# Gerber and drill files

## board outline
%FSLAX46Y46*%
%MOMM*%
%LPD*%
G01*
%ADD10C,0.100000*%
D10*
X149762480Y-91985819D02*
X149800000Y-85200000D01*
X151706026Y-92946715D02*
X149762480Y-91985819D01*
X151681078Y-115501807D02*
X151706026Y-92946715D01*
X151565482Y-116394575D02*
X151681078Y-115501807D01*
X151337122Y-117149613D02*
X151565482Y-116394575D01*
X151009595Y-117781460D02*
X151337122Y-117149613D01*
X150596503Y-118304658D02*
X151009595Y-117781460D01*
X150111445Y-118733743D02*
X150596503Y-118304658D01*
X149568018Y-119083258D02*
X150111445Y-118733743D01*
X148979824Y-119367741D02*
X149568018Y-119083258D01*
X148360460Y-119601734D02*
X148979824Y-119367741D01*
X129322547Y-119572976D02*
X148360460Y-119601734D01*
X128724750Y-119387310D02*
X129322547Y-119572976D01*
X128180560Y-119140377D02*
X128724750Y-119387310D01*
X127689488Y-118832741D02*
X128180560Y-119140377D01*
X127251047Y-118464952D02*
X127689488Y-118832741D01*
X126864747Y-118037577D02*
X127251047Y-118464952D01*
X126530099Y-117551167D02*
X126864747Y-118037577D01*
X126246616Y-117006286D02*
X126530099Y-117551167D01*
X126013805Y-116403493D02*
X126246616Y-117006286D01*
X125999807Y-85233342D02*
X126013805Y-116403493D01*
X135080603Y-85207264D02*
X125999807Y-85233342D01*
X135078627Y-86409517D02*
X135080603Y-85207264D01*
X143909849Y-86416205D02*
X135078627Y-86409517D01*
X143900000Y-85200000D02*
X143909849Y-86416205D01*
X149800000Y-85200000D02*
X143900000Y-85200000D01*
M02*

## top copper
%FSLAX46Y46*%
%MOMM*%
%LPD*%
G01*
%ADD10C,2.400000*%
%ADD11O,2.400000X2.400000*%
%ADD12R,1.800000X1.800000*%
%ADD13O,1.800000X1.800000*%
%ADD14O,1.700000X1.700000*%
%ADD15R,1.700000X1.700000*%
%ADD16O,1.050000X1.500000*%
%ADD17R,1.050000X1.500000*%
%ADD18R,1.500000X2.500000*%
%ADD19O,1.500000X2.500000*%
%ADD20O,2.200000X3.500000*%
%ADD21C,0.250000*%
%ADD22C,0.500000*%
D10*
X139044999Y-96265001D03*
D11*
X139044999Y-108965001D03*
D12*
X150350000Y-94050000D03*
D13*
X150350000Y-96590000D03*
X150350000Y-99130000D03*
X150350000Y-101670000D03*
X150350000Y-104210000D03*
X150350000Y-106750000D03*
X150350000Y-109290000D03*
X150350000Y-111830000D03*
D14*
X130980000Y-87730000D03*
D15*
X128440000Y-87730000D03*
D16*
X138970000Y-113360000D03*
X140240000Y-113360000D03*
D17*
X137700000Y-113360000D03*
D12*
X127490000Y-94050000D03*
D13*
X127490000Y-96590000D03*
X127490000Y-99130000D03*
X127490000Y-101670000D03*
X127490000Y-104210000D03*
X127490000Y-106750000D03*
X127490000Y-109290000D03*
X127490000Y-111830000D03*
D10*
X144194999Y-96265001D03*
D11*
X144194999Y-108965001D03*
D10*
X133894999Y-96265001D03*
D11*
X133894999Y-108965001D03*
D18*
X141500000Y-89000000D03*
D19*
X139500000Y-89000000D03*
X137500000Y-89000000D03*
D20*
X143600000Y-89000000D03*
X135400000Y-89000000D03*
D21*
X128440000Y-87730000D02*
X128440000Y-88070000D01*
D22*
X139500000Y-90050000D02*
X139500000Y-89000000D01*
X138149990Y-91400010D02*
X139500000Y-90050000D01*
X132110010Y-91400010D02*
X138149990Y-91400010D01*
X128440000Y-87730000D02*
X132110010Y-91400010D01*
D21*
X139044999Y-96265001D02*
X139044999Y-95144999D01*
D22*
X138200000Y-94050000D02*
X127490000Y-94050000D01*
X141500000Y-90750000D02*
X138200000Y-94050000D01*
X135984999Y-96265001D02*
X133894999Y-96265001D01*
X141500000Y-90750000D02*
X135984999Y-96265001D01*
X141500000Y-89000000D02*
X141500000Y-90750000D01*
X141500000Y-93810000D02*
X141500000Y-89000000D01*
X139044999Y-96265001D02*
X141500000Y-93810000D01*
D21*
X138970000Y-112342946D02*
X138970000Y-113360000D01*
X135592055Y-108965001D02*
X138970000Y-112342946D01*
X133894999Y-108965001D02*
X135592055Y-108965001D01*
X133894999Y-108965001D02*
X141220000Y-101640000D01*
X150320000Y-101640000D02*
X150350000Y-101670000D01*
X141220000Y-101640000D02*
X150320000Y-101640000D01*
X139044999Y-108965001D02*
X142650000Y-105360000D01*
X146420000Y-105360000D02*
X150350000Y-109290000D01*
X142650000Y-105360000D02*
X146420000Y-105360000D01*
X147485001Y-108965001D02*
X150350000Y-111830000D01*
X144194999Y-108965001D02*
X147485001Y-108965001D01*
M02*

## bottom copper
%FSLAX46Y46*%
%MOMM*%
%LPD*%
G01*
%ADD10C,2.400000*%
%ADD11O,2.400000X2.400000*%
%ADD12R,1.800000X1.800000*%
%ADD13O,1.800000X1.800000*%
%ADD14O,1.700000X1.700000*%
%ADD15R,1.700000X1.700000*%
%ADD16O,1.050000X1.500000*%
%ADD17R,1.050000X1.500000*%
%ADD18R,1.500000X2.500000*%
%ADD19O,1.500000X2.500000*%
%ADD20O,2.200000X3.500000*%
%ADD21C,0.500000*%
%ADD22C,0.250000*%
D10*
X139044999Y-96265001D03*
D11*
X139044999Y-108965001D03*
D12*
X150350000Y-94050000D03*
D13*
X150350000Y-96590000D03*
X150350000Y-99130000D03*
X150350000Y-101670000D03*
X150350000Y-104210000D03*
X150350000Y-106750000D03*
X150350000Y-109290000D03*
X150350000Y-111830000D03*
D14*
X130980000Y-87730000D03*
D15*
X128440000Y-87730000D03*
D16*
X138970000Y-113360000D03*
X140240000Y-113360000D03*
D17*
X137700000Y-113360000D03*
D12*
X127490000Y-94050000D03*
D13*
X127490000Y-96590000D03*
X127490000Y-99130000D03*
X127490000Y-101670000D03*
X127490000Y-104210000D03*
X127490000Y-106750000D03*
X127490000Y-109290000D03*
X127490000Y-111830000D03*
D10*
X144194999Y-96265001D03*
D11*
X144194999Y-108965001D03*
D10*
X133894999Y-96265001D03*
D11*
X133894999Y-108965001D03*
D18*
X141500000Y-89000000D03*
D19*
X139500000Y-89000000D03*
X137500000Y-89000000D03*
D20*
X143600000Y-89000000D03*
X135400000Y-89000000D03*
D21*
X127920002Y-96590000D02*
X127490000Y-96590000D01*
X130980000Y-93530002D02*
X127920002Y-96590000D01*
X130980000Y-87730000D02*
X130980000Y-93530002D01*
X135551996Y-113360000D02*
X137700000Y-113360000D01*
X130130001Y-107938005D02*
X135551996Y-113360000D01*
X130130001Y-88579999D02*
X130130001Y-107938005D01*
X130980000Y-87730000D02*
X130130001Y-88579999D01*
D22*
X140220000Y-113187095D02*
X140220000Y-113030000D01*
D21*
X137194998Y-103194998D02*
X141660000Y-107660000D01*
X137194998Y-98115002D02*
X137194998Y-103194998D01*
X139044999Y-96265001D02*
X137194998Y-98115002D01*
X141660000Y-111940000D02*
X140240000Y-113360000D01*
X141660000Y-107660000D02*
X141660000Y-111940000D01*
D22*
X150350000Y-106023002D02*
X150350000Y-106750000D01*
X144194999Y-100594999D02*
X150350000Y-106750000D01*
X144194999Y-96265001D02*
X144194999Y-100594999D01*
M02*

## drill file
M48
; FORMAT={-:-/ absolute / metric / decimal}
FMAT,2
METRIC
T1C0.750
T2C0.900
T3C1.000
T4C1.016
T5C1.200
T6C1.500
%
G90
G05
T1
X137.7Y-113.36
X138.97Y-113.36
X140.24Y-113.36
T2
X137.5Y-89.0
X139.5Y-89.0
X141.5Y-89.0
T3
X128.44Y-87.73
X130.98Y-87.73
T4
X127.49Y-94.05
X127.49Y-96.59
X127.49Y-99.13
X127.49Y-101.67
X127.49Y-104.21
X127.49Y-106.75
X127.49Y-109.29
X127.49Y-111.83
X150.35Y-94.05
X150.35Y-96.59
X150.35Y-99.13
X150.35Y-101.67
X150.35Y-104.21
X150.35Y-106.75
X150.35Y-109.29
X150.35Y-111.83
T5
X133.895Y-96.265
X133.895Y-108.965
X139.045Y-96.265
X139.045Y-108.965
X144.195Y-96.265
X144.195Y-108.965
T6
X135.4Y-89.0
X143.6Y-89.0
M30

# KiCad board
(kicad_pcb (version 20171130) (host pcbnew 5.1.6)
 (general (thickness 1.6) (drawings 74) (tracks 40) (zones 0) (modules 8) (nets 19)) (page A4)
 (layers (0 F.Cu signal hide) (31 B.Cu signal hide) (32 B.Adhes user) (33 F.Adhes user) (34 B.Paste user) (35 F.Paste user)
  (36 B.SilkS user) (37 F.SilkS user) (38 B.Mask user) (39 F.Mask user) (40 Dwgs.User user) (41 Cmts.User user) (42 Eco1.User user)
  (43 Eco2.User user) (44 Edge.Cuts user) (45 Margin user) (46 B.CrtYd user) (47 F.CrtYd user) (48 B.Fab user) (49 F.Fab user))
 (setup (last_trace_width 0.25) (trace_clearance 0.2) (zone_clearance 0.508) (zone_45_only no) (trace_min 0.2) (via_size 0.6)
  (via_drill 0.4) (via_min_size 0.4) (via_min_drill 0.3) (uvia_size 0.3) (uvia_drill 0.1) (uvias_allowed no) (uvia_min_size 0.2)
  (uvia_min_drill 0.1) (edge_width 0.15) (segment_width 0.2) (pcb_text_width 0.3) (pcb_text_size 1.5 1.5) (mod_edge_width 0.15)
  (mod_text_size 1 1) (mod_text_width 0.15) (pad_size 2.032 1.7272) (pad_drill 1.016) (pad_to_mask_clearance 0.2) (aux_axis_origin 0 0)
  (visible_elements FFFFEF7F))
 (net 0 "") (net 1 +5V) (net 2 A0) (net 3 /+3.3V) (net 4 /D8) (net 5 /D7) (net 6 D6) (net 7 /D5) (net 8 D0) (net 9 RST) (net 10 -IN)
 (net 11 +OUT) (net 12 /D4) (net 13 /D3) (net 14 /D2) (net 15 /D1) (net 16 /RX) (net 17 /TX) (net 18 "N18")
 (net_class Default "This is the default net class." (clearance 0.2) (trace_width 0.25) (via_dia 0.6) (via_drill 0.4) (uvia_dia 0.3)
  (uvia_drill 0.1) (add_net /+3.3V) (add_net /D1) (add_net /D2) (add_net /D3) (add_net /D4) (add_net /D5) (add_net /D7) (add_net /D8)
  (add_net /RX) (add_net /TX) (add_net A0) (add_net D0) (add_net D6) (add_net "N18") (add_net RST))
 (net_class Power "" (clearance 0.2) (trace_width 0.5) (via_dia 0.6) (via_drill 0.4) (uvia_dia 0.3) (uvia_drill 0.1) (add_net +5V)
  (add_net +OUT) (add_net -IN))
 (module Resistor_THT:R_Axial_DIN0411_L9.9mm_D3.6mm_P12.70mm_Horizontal (layer F.Cu) (at 139.044999 96.265001 270)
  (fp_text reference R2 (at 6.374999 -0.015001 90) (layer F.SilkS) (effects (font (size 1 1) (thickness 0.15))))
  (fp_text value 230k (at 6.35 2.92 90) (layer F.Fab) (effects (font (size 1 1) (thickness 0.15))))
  (pad 1 thru_hole circle (at 0 0 270) (size 2.4 2.4) (drill 1.2) (layers *.Cu *.Mask) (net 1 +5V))
  (pad 2 thru_hole oval (at 12.7 0 270) (size 2.4 2.4) (drill 1.2) (layers *.Cu *.Mask) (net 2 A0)))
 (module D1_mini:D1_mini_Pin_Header (layer B.Cu) (at 150.35 94.05 180)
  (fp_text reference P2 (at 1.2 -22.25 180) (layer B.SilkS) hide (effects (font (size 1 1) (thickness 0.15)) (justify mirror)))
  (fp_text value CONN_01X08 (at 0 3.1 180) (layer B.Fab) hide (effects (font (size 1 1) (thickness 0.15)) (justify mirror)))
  (pad 1 thru_hole rect (at 0 0 180) (size 1.8 1.8) (drill 1.016) (layers *.Cu *.Mask B.SilkS) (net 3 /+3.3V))
  (pad 2 thru_hole oval (at 0 -2.54 180) (size 1.8 1.8) (drill 1.016) (layers *.Cu *.Mask B.SilkS) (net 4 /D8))
  (pad 3 thru_hole oval (at 0 -5.08 180) (size 1.8 1.8) (drill 1.016) (layers *.Cu *.Mask B.SilkS) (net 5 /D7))
  (pad 4 thru_hole oval (at 0 -7.62 180) (size 1.8 1.8) (drill 1.016) (layers *.Cu *.Mask B.SilkS) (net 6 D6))
  (pad 5 thru_hole oval (at 0 -10.16 180) (size 1.8 1.8) (drill 1.016) (layers *.Cu *.Mask B.SilkS) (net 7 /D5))
  (pad 6 thru_hole oval (at 0 -12.7 180) (size 1.8 1.8) (drill 1.016) (layers *.Cu *.Mask B.SilkS) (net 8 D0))
  (pad 7 thru_hole oval (at 0 -15.24 180) (size 1.8 1.8) (drill 1.016) (layers *.Cu *.Mask B.SilkS) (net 2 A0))
  (pad 8 thru_hole oval (at 0 -17.78 180) (size 1.8 1.8) (drill 1.016) (layers *.Cu *.Mask B.SilkS) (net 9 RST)))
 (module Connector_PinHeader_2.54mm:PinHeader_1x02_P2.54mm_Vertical (layer F.Cu) (at 128.44 87.73 90)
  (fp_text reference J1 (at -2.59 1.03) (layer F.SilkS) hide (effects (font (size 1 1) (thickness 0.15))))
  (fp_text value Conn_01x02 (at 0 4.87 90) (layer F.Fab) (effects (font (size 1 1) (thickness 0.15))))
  (pad 2 thru_hole oval (at 0 2.54 90) (size 1.7 1.7) (drill 1) (layers *.Cu *.Mask) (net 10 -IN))
  (pad 1 thru_hole rect (at 0 0 90) (size 1.7 1.7) (drill 1) (layers *.Cu *.Mask) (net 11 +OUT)))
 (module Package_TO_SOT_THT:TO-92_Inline (layer F.Cu) (at 137.7 113.36)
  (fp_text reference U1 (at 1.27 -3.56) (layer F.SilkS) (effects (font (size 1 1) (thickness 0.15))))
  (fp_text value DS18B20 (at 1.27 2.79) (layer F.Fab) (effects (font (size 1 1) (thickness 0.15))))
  (pad 2 thru_hole oval (at 1.27 0) (size 1.05 1.5) (drill 0.75) (layers *.Cu *.Mask) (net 6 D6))
  (pad 3 thru_hole oval (at 2.54 0) (size 1.05 1.5) (drill 0.75) (layers *.Cu *.Mask) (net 1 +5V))
  (pad 1 thru_hole rect (at 0 0) (size 1.05 1.5) (drill 0.75) (layers *.Cu *.Mask) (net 10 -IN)))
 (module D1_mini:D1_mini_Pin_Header (layer B.Cu) (at 127.49 94.05 180)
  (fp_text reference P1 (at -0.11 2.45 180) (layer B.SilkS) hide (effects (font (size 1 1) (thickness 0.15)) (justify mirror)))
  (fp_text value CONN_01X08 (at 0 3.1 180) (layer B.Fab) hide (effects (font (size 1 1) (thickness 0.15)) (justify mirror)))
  (pad 1 thru_hole rect (at 0 0 180) (size 1.8 1.8) (drill 1.016) (layers *.Cu *.Mask B.SilkS) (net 1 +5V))
  (pad 2 thru_hole oval (at 0 -2.54 180) (size 1.8 1.8) (drill 1.016) (layers *.Cu *.Mask B.SilkS) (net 10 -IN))
  (pad 3 thru_hole oval (at 0 -5.08 180) (size 1.8 1.8) (drill 1.016) (layers *.Cu *.Mask B.SilkS) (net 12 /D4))
  (pad 4 thru_hole oval (at 0 -7.62 180) (size 1.8 1.8) (drill 1.016) (layers *.Cu *.Mask B.SilkS) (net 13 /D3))
  (pad 5 thru_hole oval (at 0 -10.16 180) (size 1.8 1.8) (drill 1.016) (layers *.Cu *.Mask B.SilkS) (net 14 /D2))
  (pad 6 thru_hole oval (at 0 -12.7 180) (size 1.8 1.8) (drill 1.016) (layers *.Cu *.Mask B.SilkS) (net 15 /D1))
  (pad 7 thru_hole oval (at 0 -15.24 180) (size 1.8 1.8) (drill 1.016) (layers *.Cu *.Mask B.SilkS) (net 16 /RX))
  (pad 8 thru_hole oval (at 0 -17.78 180) (size 1.8 1.8) (drill 1.016) (layers *.Cu *.Mask B.SilkS) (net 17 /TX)))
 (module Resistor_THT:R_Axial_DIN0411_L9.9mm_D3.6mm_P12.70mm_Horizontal (layer F.Cu) (at 144.194999 96.265001 270)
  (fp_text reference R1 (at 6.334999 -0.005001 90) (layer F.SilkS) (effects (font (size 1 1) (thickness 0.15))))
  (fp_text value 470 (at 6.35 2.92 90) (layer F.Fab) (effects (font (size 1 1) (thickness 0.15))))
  (pad 1 thru_hole circle (at 0 0 270) (size 2.4 2.4) (drill 1.2) (layers *.Cu *.Mask) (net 8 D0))
  (pad 2 thru_hole oval (at 12.7 0 270) (size 2.4 2.4) (drill 1.2) (layers *.Cu *.Mask) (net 9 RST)))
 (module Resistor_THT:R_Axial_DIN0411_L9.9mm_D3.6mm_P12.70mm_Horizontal (layer F.Cu) (at 133.894999 96.265001 270)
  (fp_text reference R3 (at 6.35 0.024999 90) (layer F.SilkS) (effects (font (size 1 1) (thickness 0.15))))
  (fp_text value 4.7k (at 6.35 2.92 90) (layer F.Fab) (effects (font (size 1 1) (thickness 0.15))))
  (pad 1 thru_hole circle (at 0 0 270) (size 2.4 2.4) (drill 1.2) (layers *.Cu *.Mask) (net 1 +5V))
  (pad 2 thru_hole oval (at 12.7 0 270) (size 2.4 2.4) (drill 1.2) (layers *.Cu *.Mask) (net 6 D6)))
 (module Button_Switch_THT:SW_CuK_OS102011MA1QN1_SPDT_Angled (layer F.Cu) (at 141.5 89 180)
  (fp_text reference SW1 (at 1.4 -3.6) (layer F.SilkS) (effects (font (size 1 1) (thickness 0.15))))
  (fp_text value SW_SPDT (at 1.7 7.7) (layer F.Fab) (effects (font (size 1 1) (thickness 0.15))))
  (pad 1 thru_hole rect (at 0 0 180) (size 1.5 2.5) (drill 0.9) (layers *.Cu *.Mask) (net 1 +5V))
  (pad 2 thru_hole oval (at 2 0 180) (size 1.5 2.5) (drill 0.9) (layers *.Cu *.Mask) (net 11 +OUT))
  (pad 3 thru_hole oval (at 4 0 180) (size 1.5 2.5) (drill 0.9) (layers *.Cu *.Mask) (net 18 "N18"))
  (pad "" thru_hole oval (at -2.1 0 180) (size 2.2 3.5) (drill 1.5) (layers *.Cu *.Mask))
  (pad "" thru_hole oval (at 6.1 0 180) (size 2.2 3.5) (drill 1.5) (layers *.Cu *.Mask)))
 (gr_line (start 149.76248 91.985819) (end 149.8 85.2) (layer Edge.Cuts) (width 0.1))
 (gr_line (start 151.706026 92.946715) (end 149.76248 91.985819) (layer Edge.Cuts) (width 0.1))
 (gr_line (start 151.681078 115.501807) (end 151.706026 92.946715) (layer Edge.Cuts) (width 0.1))
 (gr_line (start 151.565482 116.394575) (end 151.681078 115.501807) (layer Edge.Cuts) (width 0.1))
 (gr_line (start 151.337122 117.149613) (end 151.565482 116.394575) (layer Edge.Cuts) (width 0.1))
 (gr_line (start 151.009595 117.78146) (end 151.337122 117.149613) (layer Edge.Cuts) (width 0.1))
 (gr_line (start 150.596503 118.304658) (end 151.009595 117.78146) (layer Edge.Cuts) (width 0.1))
 (gr_line (start 150.111445 118.733743) (end 150.596503 118.304658) (layer Edge.Cuts) (width 0.1))
 (gr_line (start 149.568018 119.083258) (end 150.111445 118.733743) (layer Edge.Cuts) (width 0.1))
 (gr_line (start 148.979824 119.367741) (end 149.568018 119.083258) (layer Edge.Cuts) (width 0.1))
 (gr_line (start 148.36046 119.601734) (end 148.979824 119.367741) (layer Edge.Cuts) (width 0.1))
 (gr_line (start 129.322547 119.572976) (end 148.36046 119.601734) (layer Edge.Cuts) (width 0.1))
 (gr_line (start 128.72475 119.38731) (end 129.322547 119.572976) (layer Edge.Cuts) (width 0.1))
 (gr_line (start 128.18056 119.140377) (end 128.72475 119.38731) (layer Edge.Cuts) (width 0.1))
 (gr_line (start 127.689488 118.832741) (end 128.18056 119.140377) (layer Edge.Cuts) (width 0.1))
 (gr_line (start 127.251047 118.464952) (end 127.689488 118.832741) (layer Edge.Cuts) (width 0.1))
 (gr_line (start 126.864747 118.037577) (end 127.251047 118.464952) (layer Edge.Cuts) (width 0.1))
 (gr_line (start 126.530099 117.551167) (end 126.864747 118.037577) (layer Edge.Cuts) (width 0.1))
 (gr_line (start 126.246616 117.006286) (end 126.530099 117.551167) (layer Edge.Cuts) (width 0.1))
 (gr_line (start 126.013805 116.403493) (end 126.246616 117.006286) (layer Edge.Cuts) (width 0.1))
 (gr_line (start 125.999807 85.233342) (end 126.013805 116.403493) (layer Edge.Cuts) (width 0.1))
 (gr_line (start 135.080603 85.207264) (end 125.999807 85.233342) (layer Edge.Cuts) (width 0.1))
 (gr_line (start 135.078627 86.409517) (end 135.080603 85.207264) (layer Edge.Cuts) (width 0.1))
 (gr_line (start 143.909849 86.416205) (end 135.078627 86.409517) (layer Edge.Cuts) (width 0.1))
 (gr_line (start 143.9 85.2) (end 143.909849 86.416205) (layer Edge.Cuts) (width 0.1))
 (gr_line (start 149.8 85.2) (end 143.9 85.2) (layer Edge.Cuts) (width 0.1))
 (segment (start 128.44 87.73) (end 128.44 88.07) (width 0.25) (layer F.Cu) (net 11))
 (segment (start 139.5 90.05) (end 139.5 89) (width 0.5) (layer F.Cu) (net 11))
 (segment (start 138.14999 91.40001) (end 139.5 90.05) (width 0.5) (layer F.Cu) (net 11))
 (segment (start 132.11001 91.40001) (end 138.14999 91.40001) (width 0.5) (layer F.Cu) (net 11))
 (segment (start 128.44 87.73) (end 132.11001 91.40001) (width 0.5) (layer F.Cu) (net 11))
 (segment (start 127.920002 96.59) (end 127.49 96.59) (width 0.5) (layer B.Cu) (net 10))
 (segment (start 130.98 93.530002) (end 127.920002 96.59) (width 0.5) (layer B.Cu) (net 10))
 (segment (start 130.98 87.73) (end 130.98 93.530002) (width 0.5) (layer B.Cu) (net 10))
 (segment (start 135.551996 113.36) (end 137.7 113.36) (width 0.5) (layer B.Cu) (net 10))
 (segment (start 130.130001 107.938005) (end 135.551996 113.36) (width 0.5) (layer B.Cu) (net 10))
 (segment (start 130.130001 88.579999) (end 130.130001 107.938005) (width 0.5) (layer B.Cu) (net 10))
 (segment (start 130.98 87.73) (end 130.130001 88.579999) (width 0.5) (layer B.Cu) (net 10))
 (segment (start 140.22 113.187095) (end 140.22 113.03) (width 0.25) (layer B.Cu) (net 1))
 (segment (start 139.044999 96.265001) (end 139.044999 95.144999) (width 0.25) (layer F.Cu) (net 1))
 (segment (start 138.2 94.05) (end 127.49 94.05) (width 0.5) (layer F.Cu) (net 1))
 (segment (start 141.5 90.75) (end 138.2 94.05) (width 0.5) (layer F.Cu) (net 1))
 (segment (start 135.984999 96.265001) (end 133.894999 96.265001) (width 0.5) (layer F.Cu) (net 1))
 (segment (start 141.5 90.75) (end 135.984999 96.265001) (width 0.5) (layer F.Cu) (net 1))
 (segment (start 141.5 89) (end 141.5 90.75) (width 0.5) (layer F.Cu) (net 1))
 (segment (start 141.5 93.81) (end 141.5 89) (width 0.5) (layer F.Cu) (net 1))
 (segment (start 139.044999 96.265001) (end 141.5 93.81) (width 0.5) (layer F.Cu) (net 1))
 (segment (start 137.194998 103.194998) (end 141.66 107.66) (width 0.5) (layer B.Cu) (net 1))
 (segment (start 137.194998 98.115002) (end 137.194998 103.194998) (width 0.5) (layer B.Cu) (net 1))
 (segment (start 139.044999 96.265001) (end 137.194998 98.115002) (width 0.5) (layer B.Cu) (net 1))
 (segment (start 141.66 111.94) (end 140.24 113.36) (width 0.5) (layer B.Cu) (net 1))
 (segment (start 141.66 107.66) (end 141.66 111.94) (width 0.5) (layer B.Cu) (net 1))
 (segment (start 138.97 112.342946) (end 138.97 113.36) (width 0.25) (layer F.Cu) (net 6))
 (segment (start 135.592055 108.965001) (end 138.97 112.342946) (width 0.25) (layer F.Cu) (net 6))
 (segment (start 133.894999 108.965001) (end 135.592055 108.965001) (width 0.25) (layer F.Cu) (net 6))
 (segment (start 133.894999 108.965001) (end 141.22 101.64) (width 0.25) (layer F.Cu) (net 6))
 (segment (start 150.32 101.64) (end 150.35 101.67) (width 0.25) (layer F.Cu) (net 6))
 (segment (start 141.22 101.64) (end 150.32 101.64) (width 0.25) (layer F.Cu) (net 6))
 (segment (start 150.35 106.023002) (end 150.35 106.75) (width 0.25) (layer B.Cu) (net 8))
 (segment (start 144.194999 100.594999) (end 150.35 106.75) (width 0.25) (layer B.Cu) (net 8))
 (segment (start 144.194999 96.265001) (end 144.194999 100.594999) (width 0.25) (layer B.Cu) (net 8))
 (segment (start 139.044999 108.965001) (end 142.65 105.36) (width 0.25) (layer F.Cu) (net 2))
 (segment (start 146.42 105.36) (end 150.35 109.29) (width 0.25) (layer F.Cu) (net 2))
 (segment (start 142.65 105.36) (end 146.42 105.36) (width 0.25) (layer F.Cu) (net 2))
 (segment (start 147.485001 108.965001) (end 150.35 111.83) (width 0.25) (layer F.Cu) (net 9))
 (segment (start 144.194999 108.965001) (end 147.485001 108.965001) (width 0.25) (layer F.Cu) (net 9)))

